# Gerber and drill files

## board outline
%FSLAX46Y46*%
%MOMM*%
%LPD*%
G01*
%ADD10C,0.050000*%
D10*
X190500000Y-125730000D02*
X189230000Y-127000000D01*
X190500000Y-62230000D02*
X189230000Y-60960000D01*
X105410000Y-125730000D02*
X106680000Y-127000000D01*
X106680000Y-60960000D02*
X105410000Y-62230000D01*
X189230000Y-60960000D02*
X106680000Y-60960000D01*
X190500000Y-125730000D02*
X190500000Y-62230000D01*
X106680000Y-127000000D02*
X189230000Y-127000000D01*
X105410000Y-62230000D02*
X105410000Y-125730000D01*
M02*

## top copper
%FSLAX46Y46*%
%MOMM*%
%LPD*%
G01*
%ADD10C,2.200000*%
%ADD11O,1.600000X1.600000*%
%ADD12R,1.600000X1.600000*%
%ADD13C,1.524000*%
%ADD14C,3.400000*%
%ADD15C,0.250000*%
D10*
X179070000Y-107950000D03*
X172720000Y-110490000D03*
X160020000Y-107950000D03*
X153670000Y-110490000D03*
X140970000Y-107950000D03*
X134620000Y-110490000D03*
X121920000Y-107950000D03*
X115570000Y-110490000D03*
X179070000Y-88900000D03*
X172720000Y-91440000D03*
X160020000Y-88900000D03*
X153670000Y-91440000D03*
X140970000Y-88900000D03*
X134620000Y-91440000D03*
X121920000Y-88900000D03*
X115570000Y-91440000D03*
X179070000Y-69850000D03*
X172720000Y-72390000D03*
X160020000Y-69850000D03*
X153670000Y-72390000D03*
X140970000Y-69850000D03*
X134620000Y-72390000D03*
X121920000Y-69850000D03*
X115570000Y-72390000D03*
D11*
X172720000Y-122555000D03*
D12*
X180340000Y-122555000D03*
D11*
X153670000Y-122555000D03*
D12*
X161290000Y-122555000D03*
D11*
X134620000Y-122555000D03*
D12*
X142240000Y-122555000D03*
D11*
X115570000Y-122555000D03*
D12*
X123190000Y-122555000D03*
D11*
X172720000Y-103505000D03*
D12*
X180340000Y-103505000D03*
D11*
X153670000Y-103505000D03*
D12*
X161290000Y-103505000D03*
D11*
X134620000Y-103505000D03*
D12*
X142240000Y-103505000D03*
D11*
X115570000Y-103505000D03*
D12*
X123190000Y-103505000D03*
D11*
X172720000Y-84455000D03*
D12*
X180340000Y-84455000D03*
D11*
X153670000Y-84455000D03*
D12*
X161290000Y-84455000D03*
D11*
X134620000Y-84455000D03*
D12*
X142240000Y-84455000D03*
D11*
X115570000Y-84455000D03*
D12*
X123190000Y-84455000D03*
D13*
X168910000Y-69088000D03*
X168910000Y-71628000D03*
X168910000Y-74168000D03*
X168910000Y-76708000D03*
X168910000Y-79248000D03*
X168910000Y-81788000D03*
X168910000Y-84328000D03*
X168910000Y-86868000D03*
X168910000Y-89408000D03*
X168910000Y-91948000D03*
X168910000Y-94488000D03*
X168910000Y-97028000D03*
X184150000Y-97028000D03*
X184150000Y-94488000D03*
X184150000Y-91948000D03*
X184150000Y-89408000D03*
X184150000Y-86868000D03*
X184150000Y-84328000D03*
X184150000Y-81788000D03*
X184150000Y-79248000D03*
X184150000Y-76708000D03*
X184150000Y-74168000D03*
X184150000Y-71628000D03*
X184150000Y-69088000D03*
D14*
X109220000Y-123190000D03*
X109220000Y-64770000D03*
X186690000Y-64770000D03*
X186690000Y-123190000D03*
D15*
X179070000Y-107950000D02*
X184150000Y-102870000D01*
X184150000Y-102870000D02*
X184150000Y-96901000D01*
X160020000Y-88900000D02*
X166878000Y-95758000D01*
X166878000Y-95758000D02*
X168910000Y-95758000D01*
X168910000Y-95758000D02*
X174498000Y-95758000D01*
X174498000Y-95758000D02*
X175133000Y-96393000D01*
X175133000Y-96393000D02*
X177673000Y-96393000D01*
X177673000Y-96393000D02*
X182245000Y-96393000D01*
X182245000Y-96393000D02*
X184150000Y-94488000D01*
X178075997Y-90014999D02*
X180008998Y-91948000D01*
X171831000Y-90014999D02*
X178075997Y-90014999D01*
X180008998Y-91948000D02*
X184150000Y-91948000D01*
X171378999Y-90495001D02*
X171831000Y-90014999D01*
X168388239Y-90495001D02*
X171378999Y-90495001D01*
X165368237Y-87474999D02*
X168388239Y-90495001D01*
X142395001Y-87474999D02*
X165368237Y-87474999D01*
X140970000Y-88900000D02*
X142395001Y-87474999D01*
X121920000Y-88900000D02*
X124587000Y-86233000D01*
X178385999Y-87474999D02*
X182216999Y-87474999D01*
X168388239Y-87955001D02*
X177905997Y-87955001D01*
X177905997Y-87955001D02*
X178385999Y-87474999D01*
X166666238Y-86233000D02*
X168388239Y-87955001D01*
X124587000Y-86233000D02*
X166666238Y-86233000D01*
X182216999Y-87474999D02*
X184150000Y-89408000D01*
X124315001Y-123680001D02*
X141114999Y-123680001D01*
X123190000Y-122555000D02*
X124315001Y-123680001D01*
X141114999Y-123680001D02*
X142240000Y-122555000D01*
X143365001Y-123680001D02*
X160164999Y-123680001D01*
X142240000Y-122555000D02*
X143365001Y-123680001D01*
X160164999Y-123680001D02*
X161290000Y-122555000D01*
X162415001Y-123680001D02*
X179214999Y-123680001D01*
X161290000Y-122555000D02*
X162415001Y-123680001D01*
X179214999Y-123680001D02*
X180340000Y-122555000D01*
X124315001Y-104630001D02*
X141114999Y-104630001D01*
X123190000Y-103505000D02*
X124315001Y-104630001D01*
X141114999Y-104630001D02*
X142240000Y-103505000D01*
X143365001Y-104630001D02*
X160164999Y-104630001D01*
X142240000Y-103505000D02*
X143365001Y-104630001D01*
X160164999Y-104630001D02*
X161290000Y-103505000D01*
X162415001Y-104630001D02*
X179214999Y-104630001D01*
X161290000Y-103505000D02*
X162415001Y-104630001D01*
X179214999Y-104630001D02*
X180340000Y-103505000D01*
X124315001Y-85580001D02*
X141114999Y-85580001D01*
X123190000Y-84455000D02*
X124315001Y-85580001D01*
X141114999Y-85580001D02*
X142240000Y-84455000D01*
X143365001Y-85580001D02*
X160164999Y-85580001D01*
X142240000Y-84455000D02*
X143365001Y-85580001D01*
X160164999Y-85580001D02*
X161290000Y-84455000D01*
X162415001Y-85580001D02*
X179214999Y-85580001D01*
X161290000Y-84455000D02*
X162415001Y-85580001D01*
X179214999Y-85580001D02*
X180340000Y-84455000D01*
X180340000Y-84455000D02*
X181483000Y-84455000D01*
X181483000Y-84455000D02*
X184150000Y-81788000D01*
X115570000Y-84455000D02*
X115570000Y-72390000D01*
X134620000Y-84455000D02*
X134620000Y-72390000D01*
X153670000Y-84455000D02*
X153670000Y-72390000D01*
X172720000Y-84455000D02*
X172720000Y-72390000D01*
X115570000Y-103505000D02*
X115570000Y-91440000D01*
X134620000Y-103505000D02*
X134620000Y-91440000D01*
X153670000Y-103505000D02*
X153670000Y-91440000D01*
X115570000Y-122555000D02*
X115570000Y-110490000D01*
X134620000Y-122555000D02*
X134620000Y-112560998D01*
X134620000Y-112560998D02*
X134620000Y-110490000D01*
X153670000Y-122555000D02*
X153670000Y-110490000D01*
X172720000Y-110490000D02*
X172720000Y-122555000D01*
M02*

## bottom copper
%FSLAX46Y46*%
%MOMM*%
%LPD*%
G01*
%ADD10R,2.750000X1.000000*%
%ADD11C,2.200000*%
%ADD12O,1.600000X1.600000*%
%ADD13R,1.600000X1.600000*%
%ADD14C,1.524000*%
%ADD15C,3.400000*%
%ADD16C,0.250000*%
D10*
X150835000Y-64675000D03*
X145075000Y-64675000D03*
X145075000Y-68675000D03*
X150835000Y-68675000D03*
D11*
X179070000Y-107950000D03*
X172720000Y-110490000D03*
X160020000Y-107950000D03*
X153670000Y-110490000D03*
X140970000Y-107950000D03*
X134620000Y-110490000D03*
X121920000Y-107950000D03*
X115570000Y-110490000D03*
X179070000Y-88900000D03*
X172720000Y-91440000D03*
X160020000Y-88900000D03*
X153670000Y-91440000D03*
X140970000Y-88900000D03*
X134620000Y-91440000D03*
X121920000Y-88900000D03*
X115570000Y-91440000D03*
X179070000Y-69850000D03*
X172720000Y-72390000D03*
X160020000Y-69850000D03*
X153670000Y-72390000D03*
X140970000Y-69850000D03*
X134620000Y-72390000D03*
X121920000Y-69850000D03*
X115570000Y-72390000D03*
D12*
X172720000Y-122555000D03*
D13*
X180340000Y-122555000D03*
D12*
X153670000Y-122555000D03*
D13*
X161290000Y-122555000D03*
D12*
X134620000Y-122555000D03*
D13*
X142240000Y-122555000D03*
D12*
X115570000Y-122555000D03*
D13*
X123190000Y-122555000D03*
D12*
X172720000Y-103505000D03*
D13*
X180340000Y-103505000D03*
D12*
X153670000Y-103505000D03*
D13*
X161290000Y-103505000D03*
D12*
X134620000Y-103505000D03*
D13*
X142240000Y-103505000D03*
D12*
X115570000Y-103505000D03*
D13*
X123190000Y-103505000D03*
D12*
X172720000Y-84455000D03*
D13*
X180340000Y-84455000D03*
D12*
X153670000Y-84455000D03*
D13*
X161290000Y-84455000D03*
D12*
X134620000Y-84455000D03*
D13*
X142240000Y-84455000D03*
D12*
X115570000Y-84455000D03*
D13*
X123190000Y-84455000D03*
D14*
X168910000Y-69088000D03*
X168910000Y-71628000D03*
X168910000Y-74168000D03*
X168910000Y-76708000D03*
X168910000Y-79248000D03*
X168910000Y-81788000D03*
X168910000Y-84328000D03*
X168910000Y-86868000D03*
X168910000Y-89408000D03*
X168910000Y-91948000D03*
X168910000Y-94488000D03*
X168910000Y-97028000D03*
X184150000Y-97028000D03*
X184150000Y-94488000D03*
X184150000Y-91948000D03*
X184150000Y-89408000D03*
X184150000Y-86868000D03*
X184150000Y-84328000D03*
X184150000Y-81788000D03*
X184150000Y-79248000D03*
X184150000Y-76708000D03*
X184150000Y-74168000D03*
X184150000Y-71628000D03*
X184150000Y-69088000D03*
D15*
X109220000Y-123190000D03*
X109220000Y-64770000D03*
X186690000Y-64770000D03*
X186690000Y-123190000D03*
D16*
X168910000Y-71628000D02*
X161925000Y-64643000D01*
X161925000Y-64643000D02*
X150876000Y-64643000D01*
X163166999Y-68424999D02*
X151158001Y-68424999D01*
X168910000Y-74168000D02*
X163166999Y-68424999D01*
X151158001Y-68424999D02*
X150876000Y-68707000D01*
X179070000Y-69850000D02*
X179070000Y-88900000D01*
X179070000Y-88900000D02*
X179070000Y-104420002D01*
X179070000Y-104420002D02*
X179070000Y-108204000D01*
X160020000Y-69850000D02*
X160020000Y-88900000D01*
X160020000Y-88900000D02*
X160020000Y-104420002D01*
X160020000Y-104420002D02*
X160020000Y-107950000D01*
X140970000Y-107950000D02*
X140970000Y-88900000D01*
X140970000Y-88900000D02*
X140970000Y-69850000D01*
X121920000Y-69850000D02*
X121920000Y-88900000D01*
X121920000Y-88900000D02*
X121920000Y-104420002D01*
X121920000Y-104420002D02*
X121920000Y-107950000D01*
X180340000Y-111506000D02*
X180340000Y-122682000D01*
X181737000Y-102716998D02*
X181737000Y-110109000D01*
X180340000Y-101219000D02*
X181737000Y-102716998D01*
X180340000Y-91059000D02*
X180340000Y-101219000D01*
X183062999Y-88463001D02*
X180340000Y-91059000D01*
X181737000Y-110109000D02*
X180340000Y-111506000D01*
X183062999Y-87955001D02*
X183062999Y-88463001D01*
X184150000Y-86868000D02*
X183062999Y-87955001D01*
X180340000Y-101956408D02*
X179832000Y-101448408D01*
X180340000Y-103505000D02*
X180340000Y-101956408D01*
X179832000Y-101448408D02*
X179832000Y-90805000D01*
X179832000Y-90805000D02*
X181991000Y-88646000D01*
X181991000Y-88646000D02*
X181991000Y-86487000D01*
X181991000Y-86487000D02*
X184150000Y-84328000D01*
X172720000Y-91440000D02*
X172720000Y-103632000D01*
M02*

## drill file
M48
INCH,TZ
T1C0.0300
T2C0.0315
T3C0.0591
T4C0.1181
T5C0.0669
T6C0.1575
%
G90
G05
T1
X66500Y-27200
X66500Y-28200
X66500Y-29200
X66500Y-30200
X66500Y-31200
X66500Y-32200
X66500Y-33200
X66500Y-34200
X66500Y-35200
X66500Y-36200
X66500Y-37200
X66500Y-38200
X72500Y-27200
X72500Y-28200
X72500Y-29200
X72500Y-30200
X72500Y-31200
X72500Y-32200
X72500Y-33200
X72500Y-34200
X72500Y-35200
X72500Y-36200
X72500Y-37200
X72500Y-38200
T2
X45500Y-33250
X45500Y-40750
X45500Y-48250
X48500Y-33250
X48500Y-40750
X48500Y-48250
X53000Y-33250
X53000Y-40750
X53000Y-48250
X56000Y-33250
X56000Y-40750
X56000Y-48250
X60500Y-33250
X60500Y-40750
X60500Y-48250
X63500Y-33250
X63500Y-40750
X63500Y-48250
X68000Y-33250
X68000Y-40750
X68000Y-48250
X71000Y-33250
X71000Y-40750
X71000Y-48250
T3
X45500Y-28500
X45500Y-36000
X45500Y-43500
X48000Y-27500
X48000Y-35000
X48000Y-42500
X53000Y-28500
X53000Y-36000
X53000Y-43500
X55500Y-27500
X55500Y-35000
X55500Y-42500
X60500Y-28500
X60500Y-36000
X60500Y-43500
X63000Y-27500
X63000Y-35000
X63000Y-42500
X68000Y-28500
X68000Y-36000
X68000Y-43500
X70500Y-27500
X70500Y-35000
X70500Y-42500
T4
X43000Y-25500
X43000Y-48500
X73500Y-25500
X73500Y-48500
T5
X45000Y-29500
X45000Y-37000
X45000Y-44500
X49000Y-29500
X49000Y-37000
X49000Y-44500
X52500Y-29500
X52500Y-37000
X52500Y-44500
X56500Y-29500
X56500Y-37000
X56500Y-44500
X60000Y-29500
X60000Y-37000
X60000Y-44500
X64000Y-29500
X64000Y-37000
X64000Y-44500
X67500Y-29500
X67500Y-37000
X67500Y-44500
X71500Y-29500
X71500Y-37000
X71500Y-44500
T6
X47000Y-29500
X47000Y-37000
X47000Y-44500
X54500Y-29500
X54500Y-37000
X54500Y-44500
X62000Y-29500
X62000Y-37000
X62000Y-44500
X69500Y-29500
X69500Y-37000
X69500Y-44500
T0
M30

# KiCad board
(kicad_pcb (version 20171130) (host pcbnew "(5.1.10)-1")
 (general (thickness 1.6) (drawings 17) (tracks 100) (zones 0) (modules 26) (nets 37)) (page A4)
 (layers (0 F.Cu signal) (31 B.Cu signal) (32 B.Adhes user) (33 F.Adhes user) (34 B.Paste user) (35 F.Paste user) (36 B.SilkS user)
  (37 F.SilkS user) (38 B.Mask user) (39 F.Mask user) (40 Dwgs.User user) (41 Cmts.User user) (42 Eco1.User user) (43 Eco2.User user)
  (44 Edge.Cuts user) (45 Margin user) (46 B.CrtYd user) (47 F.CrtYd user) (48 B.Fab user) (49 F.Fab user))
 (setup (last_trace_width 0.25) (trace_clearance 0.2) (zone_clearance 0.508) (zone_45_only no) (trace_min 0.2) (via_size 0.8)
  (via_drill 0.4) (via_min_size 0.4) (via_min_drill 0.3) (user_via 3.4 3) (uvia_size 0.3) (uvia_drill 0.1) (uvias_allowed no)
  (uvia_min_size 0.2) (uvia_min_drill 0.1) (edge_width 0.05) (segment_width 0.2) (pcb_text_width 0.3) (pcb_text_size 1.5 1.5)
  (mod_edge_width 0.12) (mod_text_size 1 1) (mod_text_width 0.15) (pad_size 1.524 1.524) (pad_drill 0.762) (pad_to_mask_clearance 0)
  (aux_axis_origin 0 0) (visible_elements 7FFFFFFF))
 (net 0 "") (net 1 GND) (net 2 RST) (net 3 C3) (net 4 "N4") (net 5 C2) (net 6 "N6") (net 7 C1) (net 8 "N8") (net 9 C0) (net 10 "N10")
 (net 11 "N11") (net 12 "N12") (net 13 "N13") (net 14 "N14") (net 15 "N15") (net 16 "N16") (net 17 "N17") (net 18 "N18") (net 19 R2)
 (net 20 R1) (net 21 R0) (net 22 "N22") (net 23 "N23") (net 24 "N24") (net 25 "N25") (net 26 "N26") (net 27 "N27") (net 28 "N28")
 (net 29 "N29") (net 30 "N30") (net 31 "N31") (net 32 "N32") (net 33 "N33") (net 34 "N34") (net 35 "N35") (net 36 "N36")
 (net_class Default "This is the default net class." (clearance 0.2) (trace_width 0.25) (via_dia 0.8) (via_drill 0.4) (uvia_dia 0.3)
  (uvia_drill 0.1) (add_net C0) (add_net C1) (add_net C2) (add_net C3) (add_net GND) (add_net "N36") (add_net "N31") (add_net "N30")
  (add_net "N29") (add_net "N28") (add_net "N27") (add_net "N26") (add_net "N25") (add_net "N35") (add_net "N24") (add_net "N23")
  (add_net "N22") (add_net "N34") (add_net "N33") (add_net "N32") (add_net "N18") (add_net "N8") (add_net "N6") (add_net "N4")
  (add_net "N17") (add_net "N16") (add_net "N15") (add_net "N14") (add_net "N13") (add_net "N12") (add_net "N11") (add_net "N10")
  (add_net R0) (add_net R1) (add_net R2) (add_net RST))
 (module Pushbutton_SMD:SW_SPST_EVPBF (layer B.Cu) (at 147.955 66.675)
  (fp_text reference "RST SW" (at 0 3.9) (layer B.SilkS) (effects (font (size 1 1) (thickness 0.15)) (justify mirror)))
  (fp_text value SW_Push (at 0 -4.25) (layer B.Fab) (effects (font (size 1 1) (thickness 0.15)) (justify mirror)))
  (pad 2 smd rect (at 2.88 -2) (size 2.75 1) (layers B.Cu B.Paste B.Mask) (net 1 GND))
  (pad 2 smd rect (at -2.88 -2) (size 2.75 1) (layers B.Cu B.Paste B.Mask) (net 1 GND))
  (pad 1 smd rect (at -2.88 2) (size 2.75 1) (layers B.Cu B.Paste B.Mask) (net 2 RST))
  (pad 1 smd rect (at 2.88 2) (size 2.75 1) (layers B.Cu B.Paste B.Mask) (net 2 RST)))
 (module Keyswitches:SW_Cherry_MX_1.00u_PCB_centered (layer F.Cu) (at 176.53 113.03)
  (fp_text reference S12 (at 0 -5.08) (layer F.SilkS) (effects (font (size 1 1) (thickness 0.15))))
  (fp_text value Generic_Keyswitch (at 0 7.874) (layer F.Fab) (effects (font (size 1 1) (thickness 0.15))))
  (pad 1 thru_hole circle (at 2.54 -5.08) (size 2.2 2.2) (drill 1.5) (layers *.Cu *.Mask) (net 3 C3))
  (pad 2 thru_hole circle (at -3.81 -2.54) (size 2.2 2.2) (drill 1.5) (layers *.Cu *.Mask) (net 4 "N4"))
  (pad "" np_thru_hole circle (at 0 0) (size 4 4) (drill 4) (layers *.Cu *.Mask))
  (pad "" np_thru_hole circle (at -5.08 0) (size 1.7 1.7) (drill 1.7) (layers *.Cu *.Mask))
  (pad "" np_thru_hole circle (at 5.08 0) (size 1.7 1.7) (drill 1.7) (layers *.Cu *.Mask)))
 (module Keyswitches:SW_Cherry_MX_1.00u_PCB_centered (layer F.Cu) (at 157.48 113.03)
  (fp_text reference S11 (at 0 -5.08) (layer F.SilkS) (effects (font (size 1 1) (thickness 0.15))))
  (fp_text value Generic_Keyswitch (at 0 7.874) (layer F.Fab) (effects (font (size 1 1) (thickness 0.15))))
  (pad 1 thru_hole circle (at 2.54 -5.08) (size 2.2 2.2) (drill 1.5) (layers *.Cu *.Mask) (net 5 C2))
  (pad 2 thru_hole circle (at -3.81 -2.54) (size 2.2 2.2) (drill 1.5) (layers *.Cu *.Mask) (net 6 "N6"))
  (pad "" np_thru_hole circle (at 0 0) (size 4 4) (drill 4) (layers *.Cu *.Mask))
  (pad "" np_thru_hole circle (at -5.08 0) (size 1.7 1.7) (drill 1.7) (layers *.Cu *.Mask))
  (pad "" np_thru_hole circle (at 5.08 0) (size 1.7 1.7) (drill 1.7) (layers *.Cu *.Mask)))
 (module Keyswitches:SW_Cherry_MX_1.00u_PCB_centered (layer F.Cu) (at 138.43 113.03)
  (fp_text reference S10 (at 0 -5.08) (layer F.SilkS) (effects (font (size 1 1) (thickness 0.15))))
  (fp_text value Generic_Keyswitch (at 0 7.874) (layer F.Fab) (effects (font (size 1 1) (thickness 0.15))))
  (pad 1 thru_hole circle (at 2.54 -5.08) (size 2.2 2.2) (drill 1.5) (layers *.Cu *.Mask) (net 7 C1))
  (pad 2 thru_hole circle (at -3.81 -2.54) (size 2.2 2.2) (drill 1.5) (layers *.Cu *.Mask) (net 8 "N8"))
  (pad "" np_thru_hole circle (at 0 0) (size 4 4) (drill 4) (layers *.Cu *.Mask))
  (pad "" np_thru_hole circle (at -5.08 0) (size 1.7 1.7) (drill 1.7) (layers *.Cu *.Mask))
  (pad "" np_thru_hole circle (at 5.08 0) (size 1.7 1.7) (drill 1.7) (layers *.Cu *.Mask)))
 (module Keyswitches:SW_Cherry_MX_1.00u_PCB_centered (layer F.Cu) (at 119.38 113.03)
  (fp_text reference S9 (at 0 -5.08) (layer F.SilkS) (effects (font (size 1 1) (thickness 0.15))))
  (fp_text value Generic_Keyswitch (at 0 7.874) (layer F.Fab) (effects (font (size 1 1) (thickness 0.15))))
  (pad 1 thru_hole circle (at 2.54 -5.08) (size 2.2 2.2) (drill 1.5) (layers *.Cu *.Mask) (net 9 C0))
  (pad 2 thru_hole circle (at -3.81 -2.54) (size 2.2 2.2) (drill 1.5) (layers *.Cu *.Mask) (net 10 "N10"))
  (pad "" np_thru_hole circle (at 0 0) (size 4 4) (drill 4) (layers *.Cu *.Mask))
  (pad "" np_thru_hole circle (at -5.08 0) (size 1.7 1.7) (drill 1.7) (layers *.Cu *.Mask))
  (pad "" np_thru_hole circle (at 5.08 0) (size 1.7 1.7) (drill 1.7) (layers *.Cu *.Mask)))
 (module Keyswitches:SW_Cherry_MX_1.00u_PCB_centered (layer F.Cu) (at 176.53 93.98)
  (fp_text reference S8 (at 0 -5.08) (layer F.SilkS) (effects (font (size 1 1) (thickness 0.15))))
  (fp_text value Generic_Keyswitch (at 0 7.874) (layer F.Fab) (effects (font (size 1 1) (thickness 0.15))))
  (pad 1 thru_hole circle (at 2.54 -5.08) (size 2.2 2.2) (drill 1.5) (layers *.Cu *.Mask) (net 3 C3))
  (pad 2 thru_hole circle (at -3.81 -2.54) (size 2.2 2.2) (drill 1.5) (layers *.Cu *.Mask) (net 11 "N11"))
  (pad "" np_thru_hole circle (at 0 0) (size 4 4) (drill 4) (layers *.Cu *.Mask))
  (pad "" np_thru_hole circle (at -5.08 0) (size 1.7 1.7) (drill 1.7) (layers *.Cu *.Mask))
  (pad "" np_thru_hole circle (at 5.08 0) (size 1.7 1.7) (drill 1.7) (layers *.Cu *.Mask)))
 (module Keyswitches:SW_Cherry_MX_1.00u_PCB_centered (layer F.Cu) (at 157.48 93.98)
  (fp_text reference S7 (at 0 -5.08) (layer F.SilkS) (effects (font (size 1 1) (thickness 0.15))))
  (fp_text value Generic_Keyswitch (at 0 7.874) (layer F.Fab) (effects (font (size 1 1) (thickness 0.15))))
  (pad 1 thru_hole circle (at 2.54 -5.08) (size 2.2 2.2) (drill 1.5) (layers *.Cu *.Mask) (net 5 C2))
  (pad 2 thru_hole circle (at -3.81 -2.54) (size 2.2 2.2) (drill 1.5) (layers *.Cu *.Mask) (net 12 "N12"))
  (pad "" np_thru_hole circle (at 0 0) (size 4 4) (drill 4) (layers *.Cu *.Mask))
  (pad "" np_thru_hole circle (at -5.08 0) (size 1.7 1.7) (drill 1.7) (layers *.Cu *.Mask))
  (pad "" np_thru_hole circle (at 5.08 0) (size 1.7 1.7) (drill 1.7) (layers *.Cu *.Mask)))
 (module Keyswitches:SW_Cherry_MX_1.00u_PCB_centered (layer F.Cu) (at 138.43 93.98)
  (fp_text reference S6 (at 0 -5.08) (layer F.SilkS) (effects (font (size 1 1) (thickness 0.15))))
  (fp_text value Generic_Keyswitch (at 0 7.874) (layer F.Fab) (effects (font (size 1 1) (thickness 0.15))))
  (pad 1 thru_hole circle (at 2.54 -5.08) (size 2.2 2.2) (drill 1.5) (layers *.Cu *.Mask) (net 7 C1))
  (pad 2 thru_hole circle (at -3.81 -2.54) (size 2.2 2.2) (drill 1.5) (layers *.Cu *.Mask) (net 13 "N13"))
  (pad "" np_thru_hole circle (at 0 0) (size 4 4) (drill 4) (layers *.Cu *.Mask))
  (pad "" np_thru_hole circle (at -5.08 0) (size 1.7 1.7) (drill 1.7) (layers *.Cu *.Mask))
  (pad "" np_thru_hole circle (at 5.08 0) (size 1.7 1.7) (drill 1.7) (layers *.Cu *.Mask)))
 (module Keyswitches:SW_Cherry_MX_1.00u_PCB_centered (layer F.Cu) (at 119.38 93.98)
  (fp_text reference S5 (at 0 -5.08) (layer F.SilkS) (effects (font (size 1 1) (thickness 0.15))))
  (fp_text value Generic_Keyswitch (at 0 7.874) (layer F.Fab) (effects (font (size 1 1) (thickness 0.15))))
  (pad 1 thru_hole circle (at 2.54 -5.08) (size 2.2 2.2) (drill 1.5) (layers *.Cu *.Mask) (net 9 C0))
  (pad 2 thru_hole circle (at -3.81 -2.54) (size 2.2 2.2) (drill 1.5) (layers *.Cu *.Mask) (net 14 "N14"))
  (pad "" np_thru_hole circle (at 0 0) (size 4 4) (drill 4) (layers *.Cu *.Mask))
  (pad "" np_thru_hole circle (at -5.08 0) (size 1.7 1.7) (drill 1.7) (layers *.Cu *.Mask))
  (pad "" np_thru_hole circle (at 5.08 0) (size 1.7 1.7) (drill 1.7) (layers *.Cu *.Mask)))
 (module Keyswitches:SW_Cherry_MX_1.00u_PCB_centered (layer F.Cu) (at 176.53 74.93)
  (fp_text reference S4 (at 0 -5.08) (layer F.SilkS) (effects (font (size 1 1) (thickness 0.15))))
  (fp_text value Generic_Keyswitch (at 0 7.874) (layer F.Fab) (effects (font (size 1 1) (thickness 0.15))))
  (pad 1 thru_hole circle (at 2.54 -5.08) (size 2.2 2.2) (drill 1.5) (layers *.Cu *.Mask) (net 3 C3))
  (pad 2 thru_hole circle (at -3.81 -2.54) (size 2.2 2.2) (drill 1.5) (layers *.Cu *.Mask) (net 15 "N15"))
  (pad "" np_thru_hole circle (at 0 0) (size 4 4) (drill 4) (layers *.Cu *.Mask))
  (pad "" np_thru_hole circle (at -5.08 0) (size 1.7 1.7) (drill 1.7) (layers *.Cu *.Mask))
  (pad "" np_thru_hole circle (at 5.08 0) (size 1.7 1.7) (drill 1.7) (layers *.Cu *.Mask)))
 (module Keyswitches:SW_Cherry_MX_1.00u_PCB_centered (layer F.Cu) (at 157.48 74.93)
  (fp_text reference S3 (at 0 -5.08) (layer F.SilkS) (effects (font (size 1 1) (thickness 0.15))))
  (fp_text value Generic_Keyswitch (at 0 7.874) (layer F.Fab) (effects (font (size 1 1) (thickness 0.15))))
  (pad 1 thru_hole circle (at 2.54 -5.08) (size 2.2 2.2) (drill 1.5) (layers *.Cu *.Mask) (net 5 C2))
  (pad 2 thru_hole circle (at -3.81 -2.54) (size 2.2 2.2) (drill 1.5) (layers *.Cu *.Mask) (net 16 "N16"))
  (pad "" np_thru_hole circle (at 0 0) (size 4 4) (drill 4) (layers *.Cu *.Mask))
  (pad "" np_thru_hole circle (at -5.08 0) (size 1.7 1.7) (drill 1.7) (layers *.Cu *.Mask))
  (pad "" np_thru_hole circle (at 5.08 0) (size 1.7 1.7) (drill 1.7) (layers *.Cu *.Mask)))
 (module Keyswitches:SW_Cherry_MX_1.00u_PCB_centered (layer F.Cu) (at 138.43 74.93)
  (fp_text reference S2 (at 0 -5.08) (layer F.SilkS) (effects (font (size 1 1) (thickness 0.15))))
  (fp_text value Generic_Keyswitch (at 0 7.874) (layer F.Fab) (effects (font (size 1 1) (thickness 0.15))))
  (pad 1 thru_hole circle (at 2.54 -5.08) (size 2.2 2.2) (drill 1.5) (layers *.Cu *.Mask) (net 7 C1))
  (pad 2 thru_hole circle (at -3.81 -2.54) (size 2.2 2.2) (drill 1.5) (layers *.Cu *.Mask) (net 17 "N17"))
  (pad "" np_thru_hole circle (at 0 0) (size 4 4) (drill 4) (layers *.Cu *.Mask))
  (pad "" np_thru_hole circle (at -5.08 0) (size 1.7 1.7) (drill 1.7) (layers *.Cu *.Mask))
  (pad "" np_thru_hole circle (at 5.08 0) (size 1.7 1.7) (drill 1.7) (layers *.Cu *.Mask)))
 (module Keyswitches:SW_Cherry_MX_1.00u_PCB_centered (layer F.Cu) (at 119.38 74.93)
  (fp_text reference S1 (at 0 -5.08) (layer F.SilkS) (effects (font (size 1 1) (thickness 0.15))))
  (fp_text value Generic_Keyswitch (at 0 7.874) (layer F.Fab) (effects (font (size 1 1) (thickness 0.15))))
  (pad 1 thru_hole circle (at 2.54 -5.08) (size 2.2 2.2) (drill 1.5) (layers *.Cu *.Mask) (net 9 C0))
  (pad 2 thru_hole circle (at -3.81 -2.54) (size 2.2 2.2) (drill 1.5) (layers *.Cu *.Mask) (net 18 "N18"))
  (pad "" np_thru_hole circle (at 0 0) (size 4 4) (drill 4) (layers *.Cu *.Mask))
  (pad "" np_thru_hole circle (at -5.08 0) (size 1.7 1.7) (drill 1.7) (layers *.Cu *.Mask))
  (pad "" np_thru_hole circle (at 5.08 0) (size 1.7 1.7) (drill 1.7) (layers *.Cu *.Mask)))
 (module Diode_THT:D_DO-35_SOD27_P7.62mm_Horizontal (layer F.Cu) (at 180.34 122.555 180)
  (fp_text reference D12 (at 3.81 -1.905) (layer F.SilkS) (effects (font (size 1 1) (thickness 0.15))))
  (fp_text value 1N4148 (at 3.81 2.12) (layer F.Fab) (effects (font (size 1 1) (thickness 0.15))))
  (pad 2 thru_hole oval (at 7.62 0 180) (size 1.6 1.6) (drill 0.8) (layers *.Cu *.Mask) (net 4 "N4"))
  (pad 1 thru_hole rect (at 0 0 180) (size 1.6 1.6) (drill 0.8) (layers *.Cu *.Mask) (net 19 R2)))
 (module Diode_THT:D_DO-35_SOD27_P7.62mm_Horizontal (layer F.Cu) (at 161.29 122.555 180)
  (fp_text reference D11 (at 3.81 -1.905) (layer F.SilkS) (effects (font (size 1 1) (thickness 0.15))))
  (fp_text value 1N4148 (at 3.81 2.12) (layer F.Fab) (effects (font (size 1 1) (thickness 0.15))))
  (pad 2 thru_hole oval (at 7.62 0 180) (size 1.6 1.6) (drill 0.8) (layers *.Cu *.Mask) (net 6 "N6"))
  (pad 1 thru_hole rect (at 0 0 180) (size 1.6 1.6) (drill 0.8) (layers *.Cu *.Mask) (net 19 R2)))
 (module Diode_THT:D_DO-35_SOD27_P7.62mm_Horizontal (layer F.Cu) (at 142.24 122.555 180)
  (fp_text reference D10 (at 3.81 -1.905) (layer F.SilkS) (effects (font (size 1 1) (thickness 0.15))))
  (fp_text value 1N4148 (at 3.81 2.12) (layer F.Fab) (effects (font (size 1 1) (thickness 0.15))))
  (pad 2 thru_hole oval (at 7.62 0 180) (size 1.6 1.6) (drill 0.8) (layers *.Cu *.Mask) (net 8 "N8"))
  (pad 1 thru_hole rect (at 0 0 180) (size 1.6 1.6) (drill 0.8) (layers *.Cu *.Mask) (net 19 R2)))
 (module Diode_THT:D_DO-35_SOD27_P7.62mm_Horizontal (layer F.Cu) (at 123.19 122.555 180)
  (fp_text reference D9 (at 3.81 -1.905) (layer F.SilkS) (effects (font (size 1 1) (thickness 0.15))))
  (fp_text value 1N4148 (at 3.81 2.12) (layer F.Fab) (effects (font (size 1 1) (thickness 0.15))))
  (pad 2 thru_hole oval (at 7.62 0 180) (size 1.6 1.6) (drill 0.8) (layers *.Cu *.Mask) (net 10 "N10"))
  (pad 1 thru_hole rect (at 0 0 180) (size 1.6 1.6) (drill 0.8) (layers *.Cu *.Mask) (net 19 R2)))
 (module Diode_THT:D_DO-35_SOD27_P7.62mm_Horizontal (layer F.Cu) (at 180.34 103.505 180)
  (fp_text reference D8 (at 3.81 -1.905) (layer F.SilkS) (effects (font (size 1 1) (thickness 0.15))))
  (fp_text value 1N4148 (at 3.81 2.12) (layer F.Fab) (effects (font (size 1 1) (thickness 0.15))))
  (pad 2 thru_hole oval (at 7.62 0 180) (size 1.6 1.6) (drill 0.8) (layers *.Cu *.Mask) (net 11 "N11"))
  (pad 1 thru_hole rect (at 0 0 180) (size 1.6 1.6) (drill 0.8) (layers *.Cu *.Mask) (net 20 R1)))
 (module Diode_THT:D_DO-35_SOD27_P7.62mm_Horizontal (layer F.Cu) (at 161.29 103.505 180)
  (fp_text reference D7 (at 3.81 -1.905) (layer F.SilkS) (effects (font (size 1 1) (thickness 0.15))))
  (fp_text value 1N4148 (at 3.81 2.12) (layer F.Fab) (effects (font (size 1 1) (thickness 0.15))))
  (pad 2 thru_hole oval (at 7.62 0 180) (size 1.6 1.6) (drill 0.8) (layers *.Cu *.Mask) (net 12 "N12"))
  (pad 1 thru_hole rect (at 0 0 180) (size 1.6 1.6) (drill 0.8) (layers *.Cu *.Mask) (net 20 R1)))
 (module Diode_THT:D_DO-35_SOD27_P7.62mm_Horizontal (layer F.Cu) (at 142.24 103.505 180)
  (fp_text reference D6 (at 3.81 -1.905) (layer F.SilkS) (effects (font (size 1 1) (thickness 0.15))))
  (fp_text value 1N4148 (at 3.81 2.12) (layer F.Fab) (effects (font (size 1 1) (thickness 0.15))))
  (pad 2 thru_hole oval (at 7.62 0 180) (size 1.6 1.6) (drill 0.8) (layers *.Cu *.Mask) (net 13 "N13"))
  (pad 1 thru_hole rect (at 0 0 180) (size 1.6 1.6) (drill 0.8) (layers *.Cu *.Mask) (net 20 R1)))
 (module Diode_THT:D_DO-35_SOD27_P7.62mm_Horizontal (layer F.Cu) (at 123.19 103.505 180)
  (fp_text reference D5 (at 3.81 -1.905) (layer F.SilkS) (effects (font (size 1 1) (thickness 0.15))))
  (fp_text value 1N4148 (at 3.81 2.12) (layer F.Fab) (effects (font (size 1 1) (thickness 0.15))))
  (pad 2 thru_hole oval (at 7.62 0 180) (size 1.6 1.6) (drill 0.8) (layers *.Cu *.Mask) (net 14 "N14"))
  (pad 1 thru_hole rect (at 0 0 180) (size 1.6 1.6) (drill 0.8) (layers *.Cu *.Mask) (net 20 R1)))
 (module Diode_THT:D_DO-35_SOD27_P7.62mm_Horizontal (layer F.Cu) (at 180.34 84.455 180)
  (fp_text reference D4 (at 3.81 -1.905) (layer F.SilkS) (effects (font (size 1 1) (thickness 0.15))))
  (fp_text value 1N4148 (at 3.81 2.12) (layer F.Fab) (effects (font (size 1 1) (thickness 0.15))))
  (pad 2 thru_hole oval (at 7.62 0 180) (size 1.6 1.6) (drill 0.8) (layers *.Cu *.Mask) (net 15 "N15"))
  (pad 1 thru_hole rect (at 0 0 180) (size 1.6 1.6) (drill 0.8) (layers *.Cu *.Mask) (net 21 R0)))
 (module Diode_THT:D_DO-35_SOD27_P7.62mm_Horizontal (layer F.Cu) (at 161.29 84.455 180)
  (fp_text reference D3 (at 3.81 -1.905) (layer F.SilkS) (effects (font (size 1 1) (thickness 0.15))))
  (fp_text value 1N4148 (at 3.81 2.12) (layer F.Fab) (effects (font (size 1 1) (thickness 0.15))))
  (pad 2 thru_hole oval (at 7.62 0 180) (size 1.6 1.6) (drill 0.8) (layers *.Cu *.Mask) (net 16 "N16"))
  (pad 1 thru_hole rect (at 0 0 180) (size 1.6 1.6) (drill 0.8) (layers *.Cu *.Mask) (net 21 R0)))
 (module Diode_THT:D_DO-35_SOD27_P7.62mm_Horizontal (layer F.Cu) (at 142.24 84.455 180)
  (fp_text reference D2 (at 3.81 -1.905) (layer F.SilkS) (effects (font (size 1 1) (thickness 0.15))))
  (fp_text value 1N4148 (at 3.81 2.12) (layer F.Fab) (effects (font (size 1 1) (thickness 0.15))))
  (pad 2 thru_hole oval (at 7.62 0 180) (size 1.6 1.6) (drill 0.8) (layers *.Cu *.Mask) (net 17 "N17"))
  (pad 1 thru_hole rect (at 0 0 180) (size 1.6 1.6) (drill 0.8) (layers *.Cu *.Mask) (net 21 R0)))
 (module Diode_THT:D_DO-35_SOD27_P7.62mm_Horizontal (layer F.Cu) (at 123.19 84.455 180)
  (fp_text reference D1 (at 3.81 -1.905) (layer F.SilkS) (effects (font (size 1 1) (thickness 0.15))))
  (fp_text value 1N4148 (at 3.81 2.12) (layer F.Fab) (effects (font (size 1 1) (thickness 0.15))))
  (pad 2 thru_hole oval (at 7.62 0 180) (size 1.6 1.6) (drill 0.8) (layers *.Cu *.Mask) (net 18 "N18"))
  (pad 1 thru_hole rect (at 0 0 180) (size 1.6 1.6) (drill 0.8) (layers *.Cu *.Mask) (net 21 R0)))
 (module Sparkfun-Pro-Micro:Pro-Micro (layer B.Cu) (at 176.53 81.788 180)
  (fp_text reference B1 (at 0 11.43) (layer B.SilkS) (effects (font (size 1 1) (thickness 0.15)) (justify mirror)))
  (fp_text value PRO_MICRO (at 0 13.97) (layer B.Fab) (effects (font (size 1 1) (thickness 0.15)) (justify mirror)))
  (pad 24 thru_hole circle (at 7.62 12.7 180) (size 1.524 1.524) (drill 0.762) (layers *.Cu *.Mask) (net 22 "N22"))
  (pad 23 thru_hole circle (at 7.62 10.16 180) (size 1.524 1.524) (drill 0.762) (layers *.Cu *.Mask) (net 1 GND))
  (pad 22 thru_hole circle (at 7.62 7.62 180) (size 1.524 1.524) (drill 0.762) (layers *.Cu *.Mask) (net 2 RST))
  (pad 21 thru_hole circle (at 7.62 5.08 180) (size 1.524 1.524) (drill 0.762) (layers *.Cu *.Mask) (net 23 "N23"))
  (pad 20 thru_hole circle (at 7.62 2.54 180) (size 1.524 1.524) (drill 0.762) (layers *.Cu *.Mask) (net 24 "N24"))
  (pad 19 thru_hole circle (at 7.62 0 180) (size 1.524 1.524) (drill 0.762) (layers *.Cu *.Mask) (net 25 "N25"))
  (pad 18 thru_hole circle (at 7.62 -2.54 180) (size 1.524 1.524) (drill 0.762) (layers *.Cu *.Mask) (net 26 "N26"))
  (pad 17 thru_hole circle (at 7.62 -5.08 180) (size 1.524 1.524) (drill 0.762) (layers *.Cu *.Mask) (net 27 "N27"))
  (pad 16 thru_hole circle (at 7.62 -7.62 180) (size 1.524 1.524) (drill 0.762) (layers *.Cu *.Mask) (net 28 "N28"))
  (pad 15 thru_hole circle (at 7.62 -10.16 180) (size 1.524 1.524) (drill 0.762) (layers *.Cu *.Mask) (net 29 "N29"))
  (pad 14 thru_hole circle (at 7.62 -12.7 180) (size 1.524 1.524) (drill 0.762) (layers *.Cu *.Mask) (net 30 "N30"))
  (pad 13 thru_hole circle (at 7.62 -15.24 180) (size 1.524 1.524) (drill 0.762) (layers *.Cu *.Mask) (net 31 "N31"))
  (pad 12 thru_hole circle (at -7.62 -15.24 180) (size 1.524 1.524) (drill 0.762) (layers *.Cu *.Mask) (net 3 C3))
  (pad 11 thru_hole circle (at -7.62 -12.7 180) (size 1.524 1.524) (drill 0.762) (layers *.Cu *.Mask) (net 5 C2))
  (pad 10 thru_hole circle (at -7.62 -10.16 180) (size 1.524 1.524) (drill 0.762) (layers *.Cu *.Mask) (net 7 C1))
  (pad 9 thru_hole circle (at -7.62 -7.62 180) (size 1.524 1.524) (drill 0.762) (layers *.Cu *.Mask) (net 9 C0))
  (pad 8 thru_hole circle (at -7.62 -5.08 180) (size 1.524 1.524) (drill 0.762) (layers *.Cu *.Mask) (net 19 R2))
  (pad 7 thru_hole circle (at -7.62 -2.54 180) (size 1.524 1.524) (drill 0.762) (layers *.Cu *.Mask) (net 20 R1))
  (pad 6 thru_hole circle (at -7.62 0 180) (size 1.524 1.524) (drill 0.762) (layers *.Cu *.Mask) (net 21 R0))
  (pad 5 thru_hole circle (at -7.62 2.54 180) (size 1.524 1.524) (drill 0.762) (layers *.Cu *.Mask) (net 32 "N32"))
  (pad 4 thru_hole circle (at -7.62 5.08 180) (size 1.524 1.524) (drill 0.762) (layers *.Cu *.Mask) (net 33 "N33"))
  (pad 3 thru_hole circle (at -7.62 7.62 180) (size 1.524 1.524) (drill 0.762) (layers *.Cu *.Mask) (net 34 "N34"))
  (pad 2 thru_hole circle (at -7.62 10.16 180) (size 1.524 1.524) (drill 0.762) (layers *.Cu *.Mask) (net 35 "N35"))
  (pad 1 thru_hole circle (at -7.62 12.7 180) (size 1.524 1.524) (drill 0.762) (layers *.Cu *.Mask) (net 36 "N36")))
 (gr_line (start 190.5 125.73) (end 189.23 127) (layer Edge.Cuts) (width 0.05))
 (gr_line (start 190.5 62.23) (end 189.23 60.96) (layer Edge.Cuts) (width 0.05))
 (gr_line (start 105.41 125.73) (end 106.68 127) (layer Edge.Cuts) (width 0.05))
 (gr_line (start 106.68 60.96) (end 105.41 62.23) (layer Edge.Cuts) (width 0.05))
 (gr_line (start 189.23 60.96) (end 106.68 60.96) (layer Edge.Cuts) (width 0.05))
 (gr_line (start 190.5 125.73) (end 190.5 62.23) (layer Edge.Cuts) (width 0.05))
 (gr_line (start 106.68 127) (end 189.23 127) (layer Edge.Cuts) (width 0.05))
 (gr_line (start 105.41 62.23) (end 105.41 125.73) (layer Edge.Cuts) (width 0.05))
 (via (at 109.22 123.19) (size 3.4) (drill 3) (layers F.Cu B.Cu) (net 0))
 (via (at 109.22 64.77) (size 3.4) (drill 3) (layers F.Cu B.Cu) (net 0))
 (via (at 186.69 64.77) (size 3.4) (drill 3) (layers F.Cu B.Cu) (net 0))
 (via (at 186.69 123.19) (size 3.4) (drill 3) (layers F.Cu B.Cu) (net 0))
 (segment (start 168.91 71.628) (end 161.925 64.643) (width 0.25) (layer B.Cu) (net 1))
 (segment (start 161.925 64.643) (end 150.876 64.643) (width 0.25) (layer B.Cu) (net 1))
 (segment (start 163.166999 68.424999) (end 151.158001 68.424999) (width 0.25) (layer B.Cu) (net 2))
 (segment (start 168.91 74.168) (end 163.166999 68.424999) (width 0.25) (layer B.Cu) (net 2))
 (segment (start 151.158001 68.424999) (end 150.876 68.707) (width 0.25) (layer B.Cu) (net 2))
 (segment (start 179.07 107.95) (end 184.15 102.87) (width 0.25) (layer F.Cu) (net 3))
 (segment (start 184.15 102.87) (end 184.15 96.901) (width 0.25) (layer F.Cu) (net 3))
 (segment (start 179.07 69.85) (end 179.07 88.9) (width 0.25) (layer B.Cu) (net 3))
 (segment (start 179.07 88.9) (end 179.07 104.420002) (width 0.25) (layer B.Cu) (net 3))
 (segment (start 179.07 104.420002) (end 179.07 108.204) (width 0.25) (layer B.Cu) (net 3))
 (segment (start 160.02 69.85) (end 160.02 88.9) (width 0.25) (layer B.Cu) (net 5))
 (segment (start 160.02 88.9) (end 160.02 104.420002) (width 0.25) (layer B.Cu) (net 5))
 (segment (start 160.02 104.420002) (end 160.02 107.95) (width 0.25) (layer B.Cu) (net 5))
 (segment (start 160.02 88.9) (end 166.878 95.758) (width 0.25) (layer F.Cu) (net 5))
 (segment (start 166.878 95.758) (end 168.91 95.758) (width 0.25) (layer F.Cu) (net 5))
 (segment (start 168.91 95.758) (end 174.498 95.758) (width 0.25) (layer F.Cu) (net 5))
 (segment (start 174.498 95.758) (end 175.133 96.393) (width 0.25) (layer F.Cu) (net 5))
 (segment (start 175.133 96.393) (end 177.673 96.393) (width 0.25) (layer F.Cu) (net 5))
 (segment (start 177.673 96.393) (end 182.245 96.393) (width 0.25) (layer F.Cu) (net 5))
 (segment (start 182.245 96.393) (end 184.15 94.488) (width 0.25) (layer F.Cu) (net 5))
 (segment (start 140.97 107.95) (end 140.97 88.9) (width 0.25) (layer B.Cu) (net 7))
 (segment (start 140.97 88.9) (end 140.97 69.85) (width 0.25) (layer B.Cu) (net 7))
 (segment (start 178.075997 90.014999) (end 180.008998 91.948) (width 0.25) (layer F.Cu) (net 7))
 (segment (start 171.831 90.014999) (end 178.075997 90.014999) (width 0.25) (layer F.Cu) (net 7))
 (segment (start 180.008998 91.948) (end 184.15 91.948) (width 0.25) (layer F.Cu) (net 7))
 (segment (start 171.378999 90.495001) (end 171.831 90.014999) (width 0.25) (layer F.Cu) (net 7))
 (segment (start 168.388239 90.495001) (end 171.378999 90.495001) (width 0.25) (layer F.Cu) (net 7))
 (segment (start 165.368237 87.474999) (end 168.388239 90.495001) (width 0.25) (layer F.Cu) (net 7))
 (segment (start 142.395001 87.474999) (end 165.368237 87.474999) (width 0.25) (layer F.Cu) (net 7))
 (segment (start 140.97 88.9) (end 142.395001 87.474999) (width 0.25) (layer F.Cu) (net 7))
 (segment (start 121.92 69.85) (end 121.92 88.9) (width 0.25) (layer B.Cu) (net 9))
 (segment (start 121.92 88.9) (end 121.92 104.420002) (width 0.25) (layer B.Cu) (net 9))
 (segment (start 121.92 104.420002) (end 121.92 107.95) (width 0.25) (layer B.Cu) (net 9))
 (segment (start 121.92 88.9) (end 124.587 86.233) (width 0.25) (layer F.Cu) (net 9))
 (segment (start 178.385999 87.474999) (end 182.216999 87.474999) (width 0.25) (layer F.Cu) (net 9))
 (segment (start 168.388239 87.955001) (end 177.905997 87.955001) (width 0.25) (layer F.Cu) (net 9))
 (segment (start 177.905997 87.955001) (end 178.385999 87.474999) (width 0.25) (layer F.Cu) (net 9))
 (segment (start 166.666238 86.233) (end 168.388239 87.955001) (width 0.25) (layer F.Cu) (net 9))
 (segment (start 124.587 86.233) (end 166.666238 86.233) (width 0.25) (layer F.Cu) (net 9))
 (segment (start 182.216999 87.474999) (end 184.15 89.408) (width 0.25) (layer F.Cu) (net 9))
 (segment (start 124.315001 123.680001) (end 141.114999 123.680001) (width 0.25) (layer F.Cu) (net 19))
 (segment (start 123.19 122.555) (end 124.315001 123.680001) (width 0.25) (layer F.Cu) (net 19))
 (segment (start 141.114999 123.680001) (end 142.24 122.555) (width 0.25) (layer F.Cu) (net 19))
 (segment (start 143.365001 123.680001) (end 160.164999 123.680001) (width 0.25) (layer F.Cu) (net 19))
 (segment (start 142.24 122.555) (end 143.365001 123.680001) (width 0.25) (layer F.Cu) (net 19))
 (segment (start 160.164999 123.680001) (end 161.29 122.555) (width 0.25) (layer F.Cu) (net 19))
 (segment (start 162.415001 123.680001) (end 179.214999 123.680001) (width 0.25) (layer F.Cu) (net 19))
 (segment (start 161.29 122.555) (end 162.415001 123.680001) (width 0.25) (layer F.Cu) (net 19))
 (segment (start 179.214999 123.680001) (end 180.34 122.555) (width 0.25) (layer F.Cu) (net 19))
 (segment (start 180.34 111.506) (end 180.34 122.682) (width 0.25) (layer B.Cu) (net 19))
 (segment (start 181.737 102.716998) (end 181.737 110.109) (width 0.25) (layer B.Cu) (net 19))
 (segment (start 180.34 101.219) (end 181.737 102.716998) (width 0.25) (layer B.Cu) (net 19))
 (segment (start 180.34 91.059) (end 180.34 101.219) (width 0.25) (layer B.Cu) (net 19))
 (segment (start 183.062999 88.463001) (end 180.34 91.059) (width 0.25) (layer B.Cu) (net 19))
 (segment (start 181.737 110.109) (end 180.34 111.506) (width 0.25) (layer B.Cu) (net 19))
 (segment (start 183.062999 87.955001) (end 183.062999 88.463001) (width 0.25) (layer B.Cu) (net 19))
 (segment (start 184.15 86.868) (end 183.062999 87.955001) (width 0.25) (layer B.Cu) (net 19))
 (segment (start 124.315001 104.630001) (end 141.114999 104.630001) (width 0.25) (layer F.Cu) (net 20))
 (segment (start 123.19 103.505) (end 124.315001 104.630001) (width 0.25) (layer F.Cu) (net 20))
 (segment (start 141.114999 104.630001) (end 142.24 103.505) (width 0.25) (layer F.Cu) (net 20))
 (segment (start 143.365001 104.630001) (end 160.164999 104.630001) (width 0.25) (layer F.Cu) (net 20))
 (segment (start 142.24 103.505) (end 143.365001 104.630001) (width 0.25) (layer F.Cu) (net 20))
 (segment (start 160.164999 104.630001) (end 161.29 103.505) (width 0.25) (layer F.Cu) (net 20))
 (segment (start 162.415001 104.630001) (end 179.214999 104.630001) (width 0.25) (layer F.Cu) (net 20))
 (segment (start 161.29 103.505) (end 162.415001 104.630001) (width 0.25) (layer F.Cu) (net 20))
 (segment (start 179.214999 104.630001) (end 180.34 103.505) (width 0.25) (layer F.Cu) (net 20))
 (segment (start 180.34 101.956408) (end 179.832 101.448408) (width 0.25) (layer B.Cu) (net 20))
 (segment (start 180.34 103.505) (end 180.34 101.956408) (width 0.25) (layer B.Cu) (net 20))
 (segment (start 179.832 101.448408) (end 179.832 90.805) (width 0.25) (layer B.Cu) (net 20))
 (segment (start 179.832 90.805) (end 181.991 88.646) (width 0.25) (layer B.Cu) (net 20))
 (segment (start 181.991 88.646) (end 181.991 86.487) (width 0.25) (layer B.Cu) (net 20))
 (segment (start 181.991 86.487) (end 184.15 84.328) (width 0.25) (layer B.Cu) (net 20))
 (segment (start 124.315001 85.580001) (end 141.114999 85.580001) (width 0.25) (layer F.Cu) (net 21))
 (segment (start 123.19 84.455) (end 124.315001 85.580001) (width 0.25) (layer F.Cu) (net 21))
 (segment (start 141.114999 85.580001) (end 142.24 84.455) (width 0.25) (layer F.Cu) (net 21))
 (segment (start 143.365001 85.580001) (end 160.164999 85.580001) (width 0.25) (layer F.Cu) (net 21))
 (segment (start 142.24 84.455) (end 143.365001 85.580001) (width 0.25) (layer F.Cu) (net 21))
 (segment (start 160.164999 85.580001) (end 161.29 84.455) (width 0.25) (layer F.Cu) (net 21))
 (segment (start 162.415001 85.580001) (end 179.214999 85.580001) (width 0.25) (layer F.Cu) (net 21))
 (segment (start 161.29 84.455) (end 162.415001 85.580001) (width 0.25) (layer F.Cu) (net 21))
 (segment (start 179.214999 85.580001) (end 180.34 84.455) (width 0.25) (layer F.Cu) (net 21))
 (segment (start 180.34 84.455) (end 181.483 84.455) (width 0.25) (layer F.Cu) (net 21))
 (segment (start 181.483 84.455) (end 184.15 81.788) (width 0.25) (layer F.Cu) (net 21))
 (segment (start 115.57 84.455) (end 115.57 72.39) (width 0.25) (layer F.Cu) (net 18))
 (segment (start 134.62 84.455) (end 134.62 72.39) (width 0.25) (layer F.Cu) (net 17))
 (segment (start 153.67 84.455) (end 153.67 72.39) (width 0.25) (layer F.Cu) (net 16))
 (segment (start 172.72 84.455) (end 172.72 72.39) (width 0.25) (layer F.Cu) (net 15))
 (segment (start 115.57 103.505) (end 115.57 91.44) (width 0.25) (layer F.Cu) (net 14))
 (segment (start 134.62 103.505) (end 134.62 91.44) (width 0.25) (layer F.Cu) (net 13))
 (segment (start 153.67 103.505) (end 153.67 91.44) (width 0.25) (layer F.Cu) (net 12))
 (segment (start 172.72 91.44) (end 172.72 103.632) (width 0.25) (layer B.Cu) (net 11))
 (segment (start 115.57 122.555) (end 115.57 110.49) (width 0.25) (layer F.Cu) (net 10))
 (segment (start 134.62 122.555) (end 134.62 112.560998) (width 0.25) (layer F.Cu) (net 8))
 (segment (start 134.62 112.560998) (end 134.62 110.49) (width 0.25) (layer F.Cu) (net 8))
 (segment (start 153.67 122.555) (end 153.67 110.49) (width 0.25) (layer F.Cu) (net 6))
 (segment (start 172.72 110.49) (end 172.72 122.555) (width 0.25) (layer F.Cu) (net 4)))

